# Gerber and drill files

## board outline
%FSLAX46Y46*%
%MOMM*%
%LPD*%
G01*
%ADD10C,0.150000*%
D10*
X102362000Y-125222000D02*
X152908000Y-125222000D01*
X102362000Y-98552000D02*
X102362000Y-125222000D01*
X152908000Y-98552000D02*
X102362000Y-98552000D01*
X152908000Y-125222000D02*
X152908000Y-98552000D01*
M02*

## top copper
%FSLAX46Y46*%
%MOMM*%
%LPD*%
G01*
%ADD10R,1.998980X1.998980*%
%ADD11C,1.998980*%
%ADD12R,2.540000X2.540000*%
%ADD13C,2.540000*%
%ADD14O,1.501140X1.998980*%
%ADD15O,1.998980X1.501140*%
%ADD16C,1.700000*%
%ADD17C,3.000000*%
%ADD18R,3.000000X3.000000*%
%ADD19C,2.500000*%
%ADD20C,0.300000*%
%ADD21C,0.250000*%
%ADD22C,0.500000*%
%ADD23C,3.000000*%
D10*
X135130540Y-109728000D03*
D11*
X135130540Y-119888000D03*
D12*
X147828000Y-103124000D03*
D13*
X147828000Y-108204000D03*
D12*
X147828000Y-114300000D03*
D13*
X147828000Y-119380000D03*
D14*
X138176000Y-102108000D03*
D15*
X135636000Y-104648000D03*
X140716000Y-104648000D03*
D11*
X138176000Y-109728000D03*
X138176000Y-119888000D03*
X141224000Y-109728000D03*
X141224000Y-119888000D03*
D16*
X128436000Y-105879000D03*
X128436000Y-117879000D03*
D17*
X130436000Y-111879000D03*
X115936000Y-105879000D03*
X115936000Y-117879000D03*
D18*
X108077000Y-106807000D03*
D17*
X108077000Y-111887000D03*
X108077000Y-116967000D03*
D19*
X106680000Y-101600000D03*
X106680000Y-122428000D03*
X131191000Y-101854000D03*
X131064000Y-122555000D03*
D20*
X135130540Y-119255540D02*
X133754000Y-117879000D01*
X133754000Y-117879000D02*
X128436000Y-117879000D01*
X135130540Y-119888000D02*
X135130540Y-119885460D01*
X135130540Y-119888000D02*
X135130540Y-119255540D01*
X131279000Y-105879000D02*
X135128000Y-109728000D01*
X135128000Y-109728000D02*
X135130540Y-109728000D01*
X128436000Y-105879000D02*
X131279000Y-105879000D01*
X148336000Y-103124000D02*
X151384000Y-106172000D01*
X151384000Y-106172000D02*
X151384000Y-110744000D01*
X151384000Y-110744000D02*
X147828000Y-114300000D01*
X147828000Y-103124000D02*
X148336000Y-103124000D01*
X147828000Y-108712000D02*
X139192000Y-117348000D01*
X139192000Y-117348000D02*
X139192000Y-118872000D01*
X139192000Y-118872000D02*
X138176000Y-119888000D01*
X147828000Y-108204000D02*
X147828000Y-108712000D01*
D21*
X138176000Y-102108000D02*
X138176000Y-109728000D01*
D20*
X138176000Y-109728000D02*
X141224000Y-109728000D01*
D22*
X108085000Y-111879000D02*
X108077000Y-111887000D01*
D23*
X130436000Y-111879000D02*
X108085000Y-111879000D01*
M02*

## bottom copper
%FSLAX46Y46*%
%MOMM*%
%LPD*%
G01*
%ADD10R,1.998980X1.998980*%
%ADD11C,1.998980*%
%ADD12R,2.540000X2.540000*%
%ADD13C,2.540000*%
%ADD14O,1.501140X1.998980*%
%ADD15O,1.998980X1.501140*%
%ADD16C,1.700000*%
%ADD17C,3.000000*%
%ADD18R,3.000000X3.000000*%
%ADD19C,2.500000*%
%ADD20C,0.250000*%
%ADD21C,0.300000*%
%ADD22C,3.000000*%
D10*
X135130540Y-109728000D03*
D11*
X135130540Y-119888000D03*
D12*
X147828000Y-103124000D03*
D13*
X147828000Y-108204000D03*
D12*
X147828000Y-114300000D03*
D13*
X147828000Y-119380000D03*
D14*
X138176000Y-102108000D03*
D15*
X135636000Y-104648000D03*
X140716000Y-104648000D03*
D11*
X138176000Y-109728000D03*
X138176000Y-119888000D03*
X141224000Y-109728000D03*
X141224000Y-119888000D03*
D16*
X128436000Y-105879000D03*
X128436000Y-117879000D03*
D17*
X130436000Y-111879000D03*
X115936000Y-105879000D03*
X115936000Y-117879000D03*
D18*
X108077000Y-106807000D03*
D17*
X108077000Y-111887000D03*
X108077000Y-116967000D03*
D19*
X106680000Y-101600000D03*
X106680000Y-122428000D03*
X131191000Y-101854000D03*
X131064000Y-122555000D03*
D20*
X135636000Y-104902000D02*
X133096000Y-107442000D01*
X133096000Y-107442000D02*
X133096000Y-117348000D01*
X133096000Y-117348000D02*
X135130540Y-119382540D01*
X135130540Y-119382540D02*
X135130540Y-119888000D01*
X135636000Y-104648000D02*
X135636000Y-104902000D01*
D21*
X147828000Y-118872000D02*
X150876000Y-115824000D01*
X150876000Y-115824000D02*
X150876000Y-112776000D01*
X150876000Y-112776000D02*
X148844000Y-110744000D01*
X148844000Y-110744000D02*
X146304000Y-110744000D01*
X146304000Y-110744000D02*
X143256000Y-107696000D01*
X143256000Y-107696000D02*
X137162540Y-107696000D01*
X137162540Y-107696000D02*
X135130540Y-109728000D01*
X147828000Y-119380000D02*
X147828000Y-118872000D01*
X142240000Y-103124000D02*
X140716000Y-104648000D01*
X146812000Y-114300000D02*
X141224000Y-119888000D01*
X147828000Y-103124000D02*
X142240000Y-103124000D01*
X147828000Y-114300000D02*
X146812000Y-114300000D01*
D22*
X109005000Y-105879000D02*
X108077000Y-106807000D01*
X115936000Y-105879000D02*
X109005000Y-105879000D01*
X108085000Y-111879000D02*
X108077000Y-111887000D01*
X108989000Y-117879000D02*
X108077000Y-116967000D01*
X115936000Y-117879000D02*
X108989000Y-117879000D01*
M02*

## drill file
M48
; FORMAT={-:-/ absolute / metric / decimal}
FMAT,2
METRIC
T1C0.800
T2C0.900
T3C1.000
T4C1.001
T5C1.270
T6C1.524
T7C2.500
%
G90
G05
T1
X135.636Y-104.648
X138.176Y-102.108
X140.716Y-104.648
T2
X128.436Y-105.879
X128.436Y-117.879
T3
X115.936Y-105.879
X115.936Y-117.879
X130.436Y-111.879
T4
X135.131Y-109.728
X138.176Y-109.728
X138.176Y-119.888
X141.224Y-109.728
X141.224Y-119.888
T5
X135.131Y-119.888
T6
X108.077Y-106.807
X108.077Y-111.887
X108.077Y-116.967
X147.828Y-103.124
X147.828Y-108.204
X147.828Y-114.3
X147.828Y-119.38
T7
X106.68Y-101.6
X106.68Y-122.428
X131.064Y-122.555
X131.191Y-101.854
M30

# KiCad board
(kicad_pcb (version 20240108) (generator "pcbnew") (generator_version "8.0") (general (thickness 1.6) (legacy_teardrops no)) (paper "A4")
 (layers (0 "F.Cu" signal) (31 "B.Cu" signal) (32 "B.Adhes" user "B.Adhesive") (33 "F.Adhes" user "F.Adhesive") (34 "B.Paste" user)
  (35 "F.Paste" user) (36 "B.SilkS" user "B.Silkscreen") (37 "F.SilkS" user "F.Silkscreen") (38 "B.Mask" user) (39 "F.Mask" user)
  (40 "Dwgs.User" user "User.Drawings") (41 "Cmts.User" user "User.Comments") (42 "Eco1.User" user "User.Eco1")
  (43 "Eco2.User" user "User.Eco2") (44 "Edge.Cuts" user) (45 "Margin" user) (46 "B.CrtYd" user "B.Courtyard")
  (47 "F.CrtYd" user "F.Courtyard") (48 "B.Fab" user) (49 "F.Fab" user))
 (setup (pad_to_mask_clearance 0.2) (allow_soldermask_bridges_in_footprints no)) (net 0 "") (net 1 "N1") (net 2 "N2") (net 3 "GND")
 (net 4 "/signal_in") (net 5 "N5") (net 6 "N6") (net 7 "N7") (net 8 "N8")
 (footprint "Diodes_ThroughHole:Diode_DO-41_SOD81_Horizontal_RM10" (layer "F.Cu") (at 135.128 109.728 -90)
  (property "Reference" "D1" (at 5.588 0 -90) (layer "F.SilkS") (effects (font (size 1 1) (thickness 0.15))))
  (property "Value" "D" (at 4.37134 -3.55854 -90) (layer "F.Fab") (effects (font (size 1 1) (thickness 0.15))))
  (pad "1" thru_hole rect (at 0 -0.00254 90) (size 1.99898 1.99898) (drill 1.00076) (layers "*.Cu" "*.Mask" "F.SilkS")
   (remove_unused_layers no) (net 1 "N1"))
  (pad "2" thru_hole circle (at 10.16 -0.00254 90) (size 1.99898 1.99898) (drill 1.27) (layers "*.Cu" "*.Mask" "F.SilkS")
   (remove_unused_layers no) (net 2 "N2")))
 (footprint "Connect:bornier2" (layer "F.Cu") (at 147.828 105.664 -90)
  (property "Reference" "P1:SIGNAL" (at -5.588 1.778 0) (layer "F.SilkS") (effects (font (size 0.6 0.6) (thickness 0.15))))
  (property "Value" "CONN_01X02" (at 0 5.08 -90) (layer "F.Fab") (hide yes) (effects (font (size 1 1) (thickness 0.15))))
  (pad "1" thru_hole rect (at -2.54 0 270) (size 2.54 2.54) (drill 1.524) (layers "*.Cu" "*.Mask" "F.SilkS") (remove_unused_layers no)
   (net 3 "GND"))
  (pad "2" thru_hole circle (at 2.54 0 270) (size 2.54 2.54) (drill 1.524) (layers "*.Cu" "*.Mask" "F.SilkS") (remove_unused_layers no)
   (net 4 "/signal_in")))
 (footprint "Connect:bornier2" (layer "F.Cu") (at 147.828 116.84 -90)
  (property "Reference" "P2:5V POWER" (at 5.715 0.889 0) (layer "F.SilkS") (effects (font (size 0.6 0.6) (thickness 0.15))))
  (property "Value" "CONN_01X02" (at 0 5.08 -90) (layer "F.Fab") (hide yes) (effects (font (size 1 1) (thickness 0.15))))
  (pad "1" thru_hole rect (at -2.54 0 270) (size 2.54 2.54) (drill 1.524) (layers "*.Cu" "*.Mask" "F.SilkS") (remove_unused_layers no)
   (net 3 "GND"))
  (pad "2" thru_hole circle (at 2.54 0 270) (size 2.54 2.54) (drill 1.524) (layers "*.Cu" "*.Mask" "F.SilkS") (remove_unused_layers no)
   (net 1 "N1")))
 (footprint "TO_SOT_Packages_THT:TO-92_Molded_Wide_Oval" (layer "F.Cu") (at 135.636 104.648)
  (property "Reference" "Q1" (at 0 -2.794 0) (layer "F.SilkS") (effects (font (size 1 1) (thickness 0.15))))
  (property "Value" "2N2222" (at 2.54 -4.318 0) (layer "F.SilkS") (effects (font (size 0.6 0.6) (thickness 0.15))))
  (pad "1" thru_hole oval (at 2.54 -2.54 90) (size 1.99898 1.50114) (drill 0.8) (layers "*.Cu" "*.Mask" "F.SilkS") (remove_unused_layers no)
   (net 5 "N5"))
  (pad "2" thru_hole oval (at 0 0 90) (size 1.50114 1.99898) (drill 0.8) (layers "*.Cu" "*.Mask" "F.SilkS") (remove_unused_layers no)
   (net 2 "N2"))
  (pad "3" thru_hole oval (at 5.08 0 90) (size 1.50114 1.99898) (drill 0.8) (layers "*.Cu" "*.Mask" "F.SilkS") (remove_unused_layers no)
   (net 3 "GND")))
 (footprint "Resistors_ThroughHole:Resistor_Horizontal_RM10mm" (layer "F.Cu") (at 138.176 114.808 -90)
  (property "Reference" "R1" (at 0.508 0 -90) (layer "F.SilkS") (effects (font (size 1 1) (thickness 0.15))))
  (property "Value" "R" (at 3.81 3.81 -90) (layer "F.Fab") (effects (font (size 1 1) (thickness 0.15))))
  (pad "1" thru_hole circle (at -5.08 0 270) (size 1.99898 1.99898) (drill 1.00076) (layers "*.Cu" "*.SilkS" "*.Mask")
   (remove_unused_layers no) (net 5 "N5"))
  (pad "2" thru_hole circle (at 5.08 0 270) (size 1.99898 1.99898) (drill 1.00076) (layers "*.Cu" "*.SilkS" "*.Mask")
   (remove_unused_layers no) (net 4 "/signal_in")))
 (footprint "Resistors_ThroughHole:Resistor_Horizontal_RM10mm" (layer "F.Cu") (at 141.224 114.808 -90)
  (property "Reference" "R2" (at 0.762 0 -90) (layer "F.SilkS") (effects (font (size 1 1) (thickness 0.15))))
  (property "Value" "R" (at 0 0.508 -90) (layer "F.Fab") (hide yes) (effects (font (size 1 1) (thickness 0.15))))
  (pad "1" thru_hole circle (at -5.08 0 270) (size 1.99898 1.99898) (drill 1.00076) (layers "*.Cu" "*.SilkS" "*.Mask")
   (remove_unused_layers no) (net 5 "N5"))
  (pad "2" thru_hole circle (at 5.08 0 270) (size 1.99898 1.99898) (drill 1.00076) (layers "*.Cu" "*.SilkS" "*.Mask")
   (remove_unused_layers no) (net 3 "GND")))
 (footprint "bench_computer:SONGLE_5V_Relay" (layer "F.Cu") (at 122.936 111.379)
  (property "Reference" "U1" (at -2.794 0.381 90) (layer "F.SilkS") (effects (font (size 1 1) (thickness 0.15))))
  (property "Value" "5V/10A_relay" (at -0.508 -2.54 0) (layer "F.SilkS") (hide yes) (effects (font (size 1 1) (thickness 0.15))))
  (pad "1" thru_hole circle (at 5.5 -5.5) (size 1.7 1.7) (drill 0.9) (layers "*.Cu" "*.Mask" "F.SilkS") (remove_unused_layers no)
   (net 1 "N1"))
  (pad "2" thru_hole circle (at 5.5 6.5) (size 1.7 1.7) (drill 0.9) (layers "*.Cu" "*.Mask" "F.SilkS") (remove_unused_layers no)
   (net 2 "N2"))
  (pad "3" thru_hole circle (at 7.5 0.5) (size 3 3) (drill 1) (layers "*.Cu" "*.Mask" "F.SilkS") (remove_unused_layers no) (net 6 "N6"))
  (pad "4" thru_hole circle (at -7 -5.5) (size 3 3) (drill 1) (layers "*.Cu" "*.Mask" "F.SilkS") (remove_unused_layers no) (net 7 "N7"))
  (pad "5" thru_hole circle (at -7 6.5) (size 3 3) (drill 1) (layers "*.Cu" "*.Mask" "F.SilkS") (remove_unused_layers no) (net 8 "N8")))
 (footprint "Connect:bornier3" (layer "F.Cu") (at 108.077 111.887 -90)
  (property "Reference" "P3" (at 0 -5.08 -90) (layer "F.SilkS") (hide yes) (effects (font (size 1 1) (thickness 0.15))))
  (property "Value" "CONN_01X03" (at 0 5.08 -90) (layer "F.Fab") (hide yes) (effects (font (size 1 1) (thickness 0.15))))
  (pad "1" thru_hole rect (at -5.08 0 270) (size 3 3) (drill 1.524) (layers "*.Cu" "*.Mask" "F.SilkS") (remove_unused_layers no)
   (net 7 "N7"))
  (pad "2" thru_hole circle (at 0 0 270) (size 3 3) (drill 1.524) (layers "*.Cu" "*.Mask" "F.SilkS") (remove_unused_layers no) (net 6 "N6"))
  (pad "3" thru_hole circle (at 5.08 0 270) (size 3 3) (drill 1.524) (layers "*.Cu" "*.Mask" "F.SilkS") (remove_unused_layers no)
   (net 8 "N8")))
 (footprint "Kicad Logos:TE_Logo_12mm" (layer "F.Cu") (at 118.364 101.219)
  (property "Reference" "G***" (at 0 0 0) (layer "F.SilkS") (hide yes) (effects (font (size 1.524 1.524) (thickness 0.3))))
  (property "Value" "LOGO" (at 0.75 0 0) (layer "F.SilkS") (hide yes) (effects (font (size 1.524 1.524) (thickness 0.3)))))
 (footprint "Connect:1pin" (layer "F.Cu") (at 106.68 101.6)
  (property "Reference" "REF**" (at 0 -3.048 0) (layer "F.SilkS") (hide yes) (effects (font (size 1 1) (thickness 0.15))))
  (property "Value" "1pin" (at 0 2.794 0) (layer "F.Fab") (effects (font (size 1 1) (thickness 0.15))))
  (pad "1" thru_hole circle (at 0 0) (size 2.5 2.5) (drill 2.5) (layers "*.Cu" "*.Mask") (remove_unused_layers no)))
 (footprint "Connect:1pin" (layer "F.Cu") (at 106.68 122.428)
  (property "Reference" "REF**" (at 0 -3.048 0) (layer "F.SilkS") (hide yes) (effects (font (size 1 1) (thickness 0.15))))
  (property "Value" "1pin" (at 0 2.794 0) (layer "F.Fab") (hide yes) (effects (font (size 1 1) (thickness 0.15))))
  (pad "1" thru_hole circle (at 0 0) (size 2.5 2.5) (drill 2.5) (layers "*.Cu" "*.Mask") (remove_unused_layers no)))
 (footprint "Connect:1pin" (layer "F.Cu") (at 131.191 101.854)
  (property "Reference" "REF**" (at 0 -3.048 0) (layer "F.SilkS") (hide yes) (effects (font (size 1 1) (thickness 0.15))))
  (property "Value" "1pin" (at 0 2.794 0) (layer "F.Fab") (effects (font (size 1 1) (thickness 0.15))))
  (pad "1" thru_hole circle (at 0 0) (size 2.5 2.5) (drill 2.5) (layers "*.Cu" "*.Mask") (remove_unused_layers no)))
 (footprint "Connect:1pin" (layer "F.Cu") (at 131.064 122.555)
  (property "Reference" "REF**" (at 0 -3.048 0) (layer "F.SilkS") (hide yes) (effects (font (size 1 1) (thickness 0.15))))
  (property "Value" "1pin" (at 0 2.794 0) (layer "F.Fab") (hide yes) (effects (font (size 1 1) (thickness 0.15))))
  (pad "1" thru_hole circle (at 0 0) (size 2.5 2.5) (drill 2.5) (layers "*.Cu" "*.Mask") (remove_unused_layers no)))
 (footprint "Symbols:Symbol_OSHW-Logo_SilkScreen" (layer "B.Cu") (at 122.428 111.125 180)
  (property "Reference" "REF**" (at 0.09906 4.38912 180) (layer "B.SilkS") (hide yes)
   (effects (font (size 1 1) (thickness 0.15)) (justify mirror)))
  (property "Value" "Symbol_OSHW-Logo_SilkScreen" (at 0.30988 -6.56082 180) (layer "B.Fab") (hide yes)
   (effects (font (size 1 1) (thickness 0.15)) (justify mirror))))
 (gr_line (start 102.362 125.222) (end 152.908 125.222) (stroke (width 0.15) (type solid)) (layer "Edge.Cuts"))
 (gr_line (start 102.362 98.552) (end 102.362 125.222) (stroke (width 0.15) (type solid)) (layer "Edge.Cuts"))
 (gr_line (start 152.908 98.552) (end 102.362 98.552) (stroke (width 0.15) (type solid)) (layer "Edge.Cuts"))
 (gr_line (start 152.908 125.222) (end 152.908 98.552) (stroke (width 0.15) (type solid)) (layer "Edge.Cuts"))
 (segment (start 135.13054 119.25554) (end 133.754 117.879) (width 0.3) (layer "F.Cu") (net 2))
 (segment (start 133.754 117.879) (end 128.436 117.879) (width 0.3) (layer "F.Cu") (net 2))
 (segment (start 135.13054 119.888) (end 135.13054 119.88546) (width 0.3) (layer "F.Cu") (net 2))
 (segment (start 135.13054 119.888) (end 135.13054 119.25554) (width 0.3) (layer "F.Cu") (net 2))
 (segment (start 135.636 104.902) (end 133.096 107.442) (width 0.25) (layer "B.Cu") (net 2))
 (segment (start 133.096 107.442) (end 133.096 117.348) (width 0.25) (layer "B.Cu") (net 2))
 (segment (start 133.096 117.348) (end 135.13054 119.38254) (width 0.25) (layer "B.Cu") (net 2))
 (segment (start 135.13054 119.38254) (end 135.13054 119.888) (width 0.25) (layer "B.Cu") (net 2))
 (segment (start 135.636 104.648) (end 135.636 104.902) (width 0.25) (layer "B.Cu") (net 2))
 (segment (start 131.279 105.879) (end 135.128 109.728) (width 0.3) (layer "F.Cu") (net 1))
 (segment (start 135.128 109.728) (end 135.13054 109.728) (width 0.3) (layer "F.Cu") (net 1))
 (segment (start 128.436 105.879) (end 131.279 105.879) (width 0.3) (layer "F.Cu") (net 1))
 (segment (start 147.828 118.872) (end 150.876 115.824) (width 0.3) (layer "B.Cu") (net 1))
 (segment (start 150.876 115.824) (end 150.876 112.776) (width 0.3) (layer "B.Cu") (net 1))
 (segment (start 150.876 112.776) (end 148.844 110.744) (width 0.3) (layer "B.Cu") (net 1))
 (segment (start 148.844 110.744) (end 146.304 110.744) (width 0.3) (layer "B.Cu") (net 1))
 (segment (start 146.304 110.744) (end 143.256 107.696) (width 0.3) (layer "B.Cu") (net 1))
 (segment (start 143.256 107.696) (end 137.16254 107.696) (width 0.3) (layer "B.Cu") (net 1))
 (segment (start 137.16254 107.696) (end 135.13054 109.728) (width 0.3) (layer "B.Cu") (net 1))
 (segment (start 147.828 119.38) (end 147.828 118.872) (width 0.3) (layer "B.Cu") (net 1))
 (segment (start 148.336 103.124) (end 151.384 106.172) (width 0.3) (layer "F.Cu") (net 3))
 (segment (start 151.384 106.172) (end 151.384 110.744) (width 0.3) (layer "F.Cu") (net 3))
 (segment (start 151.384 110.744) (end 147.828 114.3) (width 0.3) (layer "F.Cu") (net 3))
 (segment (start 147.828 103.124) (end 148.336 103.124) (width 0.3) (layer "F.Cu") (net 3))
 (segment (start 142.24 103.124) (end 140.716 104.648) (width 0.3) (layer "B.Cu") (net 3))
 (segment (start 146.812 114.3) (end 141.224 119.888) (width 0.3) (layer "B.Cu") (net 3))
 (segment (start 147.828 103.124) (end 142.24 103.124) (width 0.3) (layer "B.Cu") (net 3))
 (segment (start 147.828 114.3) (end 146.812 114.3) (width 0.3) (layer "B.Cu") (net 3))
 (segment (start 147.828 108.712) (end 139.192 117.348) (width 0.3) (layer "F.Cu") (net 4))
 (segment (start 139.192 117.348) (end 139.192 118.872) (width 0.3) (layer "F.Cu") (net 4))
 (segment (start 139.192 118.872) (end 138.176 119.888) (width 0.3) (layer "F.Cu") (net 4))
 (segment (start 147.828 108.204) (end 147.828 108.712) (width 0.3) (layer "F.Cu") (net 4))
 (segment (start 138.176 102.108) (end 138.176 109.728) (width 0.25) (layer "F.Cu") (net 5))
 (segment (start 138.176 109.728) (end 141.224 109.728) (width 0.3) (layer "F.Cu") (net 5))
 (segment (start 109.005 105.879) (end 108.077 106.807) (width 3) (layer "B.Cu") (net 7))
 (segment (start 115.936 105.879) (end 109.005 105.879) (width 3) (layer "B.Cu") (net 7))
 (segment (start 108.085 111.879) (end 108.077 111.887) (width 0.5) (layer "F.Cu") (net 6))
 (segment (start 130.436 111.879) (end 108.085 111.879) (width 3) (layer "F.Cu") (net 6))
 (segment (start 108.085 111.879) (end 108.077 111.887) (width 3) (layer "B.Cu") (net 6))
 (segment (start 108.989 117.879) (end 108.077 116.967) (width 3) (layer "B.Cu") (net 8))
 (segment (start 115.936 117.879) (end 108.989 117.879) (width 3) (layer "B.Cu") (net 8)))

